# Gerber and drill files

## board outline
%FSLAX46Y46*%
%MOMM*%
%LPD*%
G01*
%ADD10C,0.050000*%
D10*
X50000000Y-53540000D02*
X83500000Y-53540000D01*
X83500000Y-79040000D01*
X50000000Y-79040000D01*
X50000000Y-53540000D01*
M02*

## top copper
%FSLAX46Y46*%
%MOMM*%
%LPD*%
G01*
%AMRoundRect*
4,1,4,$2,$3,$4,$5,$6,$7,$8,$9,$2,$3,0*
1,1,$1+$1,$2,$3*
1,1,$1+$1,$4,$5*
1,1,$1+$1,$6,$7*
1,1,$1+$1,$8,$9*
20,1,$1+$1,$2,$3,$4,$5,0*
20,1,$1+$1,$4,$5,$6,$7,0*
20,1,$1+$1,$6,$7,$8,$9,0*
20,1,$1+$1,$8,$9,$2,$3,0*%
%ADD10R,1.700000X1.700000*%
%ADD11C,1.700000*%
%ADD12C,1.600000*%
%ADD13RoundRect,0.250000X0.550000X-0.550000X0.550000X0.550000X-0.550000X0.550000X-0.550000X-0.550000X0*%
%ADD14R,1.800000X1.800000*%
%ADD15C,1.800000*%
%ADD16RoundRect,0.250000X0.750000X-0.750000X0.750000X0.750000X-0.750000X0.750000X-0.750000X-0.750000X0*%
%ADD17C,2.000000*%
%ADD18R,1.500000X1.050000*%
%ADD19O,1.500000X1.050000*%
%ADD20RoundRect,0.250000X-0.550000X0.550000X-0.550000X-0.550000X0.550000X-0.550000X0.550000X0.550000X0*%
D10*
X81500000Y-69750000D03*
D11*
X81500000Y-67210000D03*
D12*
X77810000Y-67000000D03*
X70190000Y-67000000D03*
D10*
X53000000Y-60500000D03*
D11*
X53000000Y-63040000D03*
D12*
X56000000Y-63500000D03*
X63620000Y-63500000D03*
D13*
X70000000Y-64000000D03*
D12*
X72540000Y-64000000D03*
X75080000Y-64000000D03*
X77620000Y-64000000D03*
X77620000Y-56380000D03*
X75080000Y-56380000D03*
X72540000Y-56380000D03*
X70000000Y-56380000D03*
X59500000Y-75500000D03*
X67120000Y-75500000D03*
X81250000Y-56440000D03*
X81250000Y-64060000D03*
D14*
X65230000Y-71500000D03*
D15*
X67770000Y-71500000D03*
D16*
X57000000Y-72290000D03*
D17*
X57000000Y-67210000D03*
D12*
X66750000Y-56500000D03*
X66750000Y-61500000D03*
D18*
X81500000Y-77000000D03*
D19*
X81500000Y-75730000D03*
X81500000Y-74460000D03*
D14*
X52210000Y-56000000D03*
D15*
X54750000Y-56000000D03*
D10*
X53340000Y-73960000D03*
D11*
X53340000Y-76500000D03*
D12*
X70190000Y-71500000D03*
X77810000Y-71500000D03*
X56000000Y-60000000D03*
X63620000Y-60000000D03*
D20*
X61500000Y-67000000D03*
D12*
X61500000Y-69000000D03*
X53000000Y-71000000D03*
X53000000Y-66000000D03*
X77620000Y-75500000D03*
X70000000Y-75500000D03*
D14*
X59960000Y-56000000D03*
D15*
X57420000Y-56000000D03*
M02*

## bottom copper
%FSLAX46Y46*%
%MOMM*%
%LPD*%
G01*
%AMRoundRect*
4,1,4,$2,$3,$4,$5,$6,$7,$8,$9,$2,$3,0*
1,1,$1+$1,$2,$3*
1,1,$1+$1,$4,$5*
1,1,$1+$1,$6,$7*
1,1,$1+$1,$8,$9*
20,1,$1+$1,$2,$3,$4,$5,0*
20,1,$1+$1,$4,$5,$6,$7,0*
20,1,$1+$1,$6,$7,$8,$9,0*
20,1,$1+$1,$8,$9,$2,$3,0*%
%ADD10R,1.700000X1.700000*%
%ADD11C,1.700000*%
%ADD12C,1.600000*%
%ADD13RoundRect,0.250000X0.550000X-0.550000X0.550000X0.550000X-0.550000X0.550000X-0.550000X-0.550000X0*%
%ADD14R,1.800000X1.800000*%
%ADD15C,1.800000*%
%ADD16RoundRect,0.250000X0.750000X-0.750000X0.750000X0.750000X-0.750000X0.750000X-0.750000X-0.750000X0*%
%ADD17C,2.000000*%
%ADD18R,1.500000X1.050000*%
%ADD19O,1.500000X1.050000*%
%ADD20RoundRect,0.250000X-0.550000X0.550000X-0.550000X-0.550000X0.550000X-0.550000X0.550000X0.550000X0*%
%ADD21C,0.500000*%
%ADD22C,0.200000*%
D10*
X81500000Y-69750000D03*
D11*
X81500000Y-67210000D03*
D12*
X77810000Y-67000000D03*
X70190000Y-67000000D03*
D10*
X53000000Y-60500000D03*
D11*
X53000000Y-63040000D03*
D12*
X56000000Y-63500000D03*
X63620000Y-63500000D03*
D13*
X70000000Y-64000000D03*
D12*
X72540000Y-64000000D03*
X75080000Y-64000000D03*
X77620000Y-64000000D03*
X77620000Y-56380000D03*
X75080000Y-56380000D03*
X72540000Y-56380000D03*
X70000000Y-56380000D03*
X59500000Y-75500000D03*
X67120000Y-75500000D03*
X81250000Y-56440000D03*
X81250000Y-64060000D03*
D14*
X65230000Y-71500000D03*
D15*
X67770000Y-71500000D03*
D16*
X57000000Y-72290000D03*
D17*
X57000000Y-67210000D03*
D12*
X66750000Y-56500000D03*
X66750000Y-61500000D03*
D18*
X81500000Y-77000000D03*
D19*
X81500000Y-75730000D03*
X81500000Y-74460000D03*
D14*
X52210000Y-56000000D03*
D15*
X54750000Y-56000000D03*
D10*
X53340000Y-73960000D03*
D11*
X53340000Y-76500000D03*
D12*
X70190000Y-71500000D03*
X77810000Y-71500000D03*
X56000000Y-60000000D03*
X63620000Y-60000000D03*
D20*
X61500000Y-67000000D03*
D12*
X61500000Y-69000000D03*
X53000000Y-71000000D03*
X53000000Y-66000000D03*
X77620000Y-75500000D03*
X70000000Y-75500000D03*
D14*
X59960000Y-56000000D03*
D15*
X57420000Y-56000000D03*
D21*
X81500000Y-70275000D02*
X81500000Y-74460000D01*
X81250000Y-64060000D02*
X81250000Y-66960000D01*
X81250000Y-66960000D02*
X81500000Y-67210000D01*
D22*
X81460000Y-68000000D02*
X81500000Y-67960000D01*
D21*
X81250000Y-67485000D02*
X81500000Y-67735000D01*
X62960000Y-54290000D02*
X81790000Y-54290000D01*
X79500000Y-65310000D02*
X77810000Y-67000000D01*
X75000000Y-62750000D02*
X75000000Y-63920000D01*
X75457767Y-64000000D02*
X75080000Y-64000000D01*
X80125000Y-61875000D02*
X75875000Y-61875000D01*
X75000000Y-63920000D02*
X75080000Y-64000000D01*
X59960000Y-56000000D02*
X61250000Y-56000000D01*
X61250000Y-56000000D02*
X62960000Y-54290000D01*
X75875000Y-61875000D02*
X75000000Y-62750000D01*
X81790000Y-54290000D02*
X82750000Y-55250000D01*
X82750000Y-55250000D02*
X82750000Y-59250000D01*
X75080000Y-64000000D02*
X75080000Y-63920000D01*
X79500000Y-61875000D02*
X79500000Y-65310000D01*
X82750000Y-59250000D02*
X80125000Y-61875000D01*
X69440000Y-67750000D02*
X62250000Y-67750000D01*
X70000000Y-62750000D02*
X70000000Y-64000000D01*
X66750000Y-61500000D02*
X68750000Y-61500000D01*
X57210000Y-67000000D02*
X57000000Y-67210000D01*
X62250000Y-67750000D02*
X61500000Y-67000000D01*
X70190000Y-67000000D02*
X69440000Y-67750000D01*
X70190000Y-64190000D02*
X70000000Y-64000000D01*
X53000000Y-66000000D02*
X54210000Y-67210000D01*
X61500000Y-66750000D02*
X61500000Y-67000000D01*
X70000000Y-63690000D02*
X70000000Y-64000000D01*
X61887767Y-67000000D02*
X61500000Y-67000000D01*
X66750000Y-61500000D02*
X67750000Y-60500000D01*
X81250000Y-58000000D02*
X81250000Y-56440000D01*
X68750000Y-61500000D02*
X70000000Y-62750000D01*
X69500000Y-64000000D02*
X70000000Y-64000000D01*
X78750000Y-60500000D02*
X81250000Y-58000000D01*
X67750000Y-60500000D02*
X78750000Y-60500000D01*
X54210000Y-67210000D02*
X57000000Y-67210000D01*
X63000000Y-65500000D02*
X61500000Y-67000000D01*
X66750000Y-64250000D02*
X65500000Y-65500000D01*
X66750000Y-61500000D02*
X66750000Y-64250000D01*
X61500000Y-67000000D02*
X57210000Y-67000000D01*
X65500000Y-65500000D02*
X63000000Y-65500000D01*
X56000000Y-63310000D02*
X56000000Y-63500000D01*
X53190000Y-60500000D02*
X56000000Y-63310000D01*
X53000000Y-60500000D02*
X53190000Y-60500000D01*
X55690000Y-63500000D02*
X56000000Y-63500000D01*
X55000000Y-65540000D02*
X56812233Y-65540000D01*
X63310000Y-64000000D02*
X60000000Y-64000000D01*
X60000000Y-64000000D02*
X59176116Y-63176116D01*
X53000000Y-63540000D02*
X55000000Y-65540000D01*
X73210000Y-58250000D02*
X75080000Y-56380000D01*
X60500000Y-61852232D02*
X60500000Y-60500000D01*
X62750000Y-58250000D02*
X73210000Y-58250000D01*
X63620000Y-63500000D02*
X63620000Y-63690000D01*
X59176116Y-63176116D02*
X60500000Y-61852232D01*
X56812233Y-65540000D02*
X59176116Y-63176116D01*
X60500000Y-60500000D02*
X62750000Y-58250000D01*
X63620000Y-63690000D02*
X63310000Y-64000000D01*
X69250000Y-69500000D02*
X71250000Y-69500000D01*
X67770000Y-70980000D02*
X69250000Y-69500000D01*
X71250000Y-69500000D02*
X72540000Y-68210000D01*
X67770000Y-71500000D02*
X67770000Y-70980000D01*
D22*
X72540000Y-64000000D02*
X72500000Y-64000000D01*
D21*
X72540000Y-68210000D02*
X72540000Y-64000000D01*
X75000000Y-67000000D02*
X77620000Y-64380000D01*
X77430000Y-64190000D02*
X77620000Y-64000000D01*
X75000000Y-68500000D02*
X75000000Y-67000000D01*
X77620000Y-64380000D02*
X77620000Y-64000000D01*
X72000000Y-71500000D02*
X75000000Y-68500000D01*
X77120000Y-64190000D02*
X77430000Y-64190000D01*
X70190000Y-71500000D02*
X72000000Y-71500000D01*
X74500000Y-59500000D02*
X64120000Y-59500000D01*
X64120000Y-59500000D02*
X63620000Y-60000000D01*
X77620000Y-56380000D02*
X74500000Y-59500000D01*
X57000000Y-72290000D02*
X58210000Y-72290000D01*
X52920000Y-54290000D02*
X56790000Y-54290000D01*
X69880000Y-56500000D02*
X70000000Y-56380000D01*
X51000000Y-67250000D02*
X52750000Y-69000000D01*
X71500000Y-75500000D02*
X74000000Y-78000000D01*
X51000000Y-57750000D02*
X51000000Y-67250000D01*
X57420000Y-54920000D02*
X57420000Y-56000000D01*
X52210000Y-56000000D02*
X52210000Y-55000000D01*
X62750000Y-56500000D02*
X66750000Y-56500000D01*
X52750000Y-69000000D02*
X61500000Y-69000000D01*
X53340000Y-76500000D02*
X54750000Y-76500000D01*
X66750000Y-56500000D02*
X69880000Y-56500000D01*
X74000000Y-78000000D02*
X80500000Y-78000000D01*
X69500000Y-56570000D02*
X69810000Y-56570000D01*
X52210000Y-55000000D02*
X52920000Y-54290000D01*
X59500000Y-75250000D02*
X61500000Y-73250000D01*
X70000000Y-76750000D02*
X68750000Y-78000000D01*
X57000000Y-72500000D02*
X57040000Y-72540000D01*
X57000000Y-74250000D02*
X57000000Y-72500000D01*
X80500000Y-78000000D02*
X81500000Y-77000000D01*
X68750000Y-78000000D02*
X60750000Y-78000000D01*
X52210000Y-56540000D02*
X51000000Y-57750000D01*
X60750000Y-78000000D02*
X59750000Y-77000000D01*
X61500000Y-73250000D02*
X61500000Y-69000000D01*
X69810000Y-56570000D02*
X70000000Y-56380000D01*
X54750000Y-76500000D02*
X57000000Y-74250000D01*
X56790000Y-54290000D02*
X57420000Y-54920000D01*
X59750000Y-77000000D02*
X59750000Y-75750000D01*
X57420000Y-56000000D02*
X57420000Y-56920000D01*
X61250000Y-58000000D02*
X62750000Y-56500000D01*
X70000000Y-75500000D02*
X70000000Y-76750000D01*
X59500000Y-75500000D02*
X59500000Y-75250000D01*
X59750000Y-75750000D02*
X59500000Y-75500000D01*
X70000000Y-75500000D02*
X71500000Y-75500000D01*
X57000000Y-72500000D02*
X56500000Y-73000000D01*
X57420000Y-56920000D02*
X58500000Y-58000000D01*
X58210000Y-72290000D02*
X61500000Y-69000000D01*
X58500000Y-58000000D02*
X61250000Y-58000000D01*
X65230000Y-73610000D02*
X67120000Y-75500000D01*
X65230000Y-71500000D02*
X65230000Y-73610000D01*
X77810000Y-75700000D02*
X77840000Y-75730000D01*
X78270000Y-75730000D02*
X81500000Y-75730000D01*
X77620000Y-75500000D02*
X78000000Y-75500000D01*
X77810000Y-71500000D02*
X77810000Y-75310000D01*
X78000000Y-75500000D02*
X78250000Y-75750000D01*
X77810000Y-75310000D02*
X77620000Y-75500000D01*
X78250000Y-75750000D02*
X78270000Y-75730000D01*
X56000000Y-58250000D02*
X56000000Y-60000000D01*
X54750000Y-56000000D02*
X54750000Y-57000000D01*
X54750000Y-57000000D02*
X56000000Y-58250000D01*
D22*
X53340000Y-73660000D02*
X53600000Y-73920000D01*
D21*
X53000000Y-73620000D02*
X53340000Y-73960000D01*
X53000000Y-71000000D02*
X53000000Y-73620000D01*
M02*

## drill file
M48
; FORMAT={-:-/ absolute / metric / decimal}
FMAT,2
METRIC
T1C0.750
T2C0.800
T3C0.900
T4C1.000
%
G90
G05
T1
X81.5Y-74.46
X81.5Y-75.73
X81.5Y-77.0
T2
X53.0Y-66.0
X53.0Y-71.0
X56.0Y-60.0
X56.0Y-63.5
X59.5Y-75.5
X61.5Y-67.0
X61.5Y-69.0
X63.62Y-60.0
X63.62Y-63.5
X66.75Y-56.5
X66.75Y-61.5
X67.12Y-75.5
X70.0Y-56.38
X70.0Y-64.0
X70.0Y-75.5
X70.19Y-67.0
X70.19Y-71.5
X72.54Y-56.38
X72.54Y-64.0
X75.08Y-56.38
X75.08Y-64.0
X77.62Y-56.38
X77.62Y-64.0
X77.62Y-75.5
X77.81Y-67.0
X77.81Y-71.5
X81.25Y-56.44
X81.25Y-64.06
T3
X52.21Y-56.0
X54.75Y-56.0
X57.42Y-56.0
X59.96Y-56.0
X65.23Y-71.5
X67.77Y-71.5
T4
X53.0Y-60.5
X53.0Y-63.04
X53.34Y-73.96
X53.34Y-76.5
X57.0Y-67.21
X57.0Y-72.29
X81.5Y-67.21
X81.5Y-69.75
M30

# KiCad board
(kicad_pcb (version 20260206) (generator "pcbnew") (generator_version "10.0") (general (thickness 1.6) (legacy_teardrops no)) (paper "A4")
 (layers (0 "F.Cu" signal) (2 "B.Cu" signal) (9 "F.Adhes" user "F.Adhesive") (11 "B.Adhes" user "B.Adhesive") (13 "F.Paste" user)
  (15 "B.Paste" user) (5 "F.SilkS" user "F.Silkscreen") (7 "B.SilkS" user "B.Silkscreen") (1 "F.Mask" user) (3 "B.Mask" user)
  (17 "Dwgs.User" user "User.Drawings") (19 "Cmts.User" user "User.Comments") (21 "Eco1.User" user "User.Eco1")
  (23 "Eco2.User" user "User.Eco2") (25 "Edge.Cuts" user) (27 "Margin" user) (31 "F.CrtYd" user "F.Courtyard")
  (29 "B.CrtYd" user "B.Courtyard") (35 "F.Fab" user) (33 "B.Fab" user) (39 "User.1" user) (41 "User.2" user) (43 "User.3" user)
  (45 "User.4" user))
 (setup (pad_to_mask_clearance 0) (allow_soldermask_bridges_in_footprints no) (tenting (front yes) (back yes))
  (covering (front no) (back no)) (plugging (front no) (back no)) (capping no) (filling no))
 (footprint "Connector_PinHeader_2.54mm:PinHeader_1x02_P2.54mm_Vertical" (layer "F.Cu") (at 81.5 69.75 180)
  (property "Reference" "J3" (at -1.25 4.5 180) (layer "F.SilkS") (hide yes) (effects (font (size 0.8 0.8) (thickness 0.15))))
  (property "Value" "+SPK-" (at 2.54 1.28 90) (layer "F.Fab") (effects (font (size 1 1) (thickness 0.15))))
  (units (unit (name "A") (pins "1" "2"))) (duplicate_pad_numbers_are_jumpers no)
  (pad "1" thru_hole rect (at 0 0 180) (size 1.7 1.7) (drill 1) (layers "*.Cu" "*.Mask") (remove_unused_layers no) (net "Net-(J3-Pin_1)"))
  (pad "2" thru_hole circle (at 0 2.54 180) (size 1.7 1.7) (drill 1) (layers "*.Cu" "*.Mask") (remove_unused_layers no)
   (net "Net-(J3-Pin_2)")))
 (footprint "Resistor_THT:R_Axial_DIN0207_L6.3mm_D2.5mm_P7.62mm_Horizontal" (layer "F.Cu") (at 77.81 67 180)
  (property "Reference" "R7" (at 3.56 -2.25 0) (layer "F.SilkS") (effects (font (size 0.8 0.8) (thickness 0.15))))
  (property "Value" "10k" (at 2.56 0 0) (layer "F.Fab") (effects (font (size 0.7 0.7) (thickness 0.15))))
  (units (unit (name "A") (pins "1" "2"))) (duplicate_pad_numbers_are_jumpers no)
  (pad "1" thru_hole circle (at 0 0 180) (size 1.6 1.6) (drill 0.8) (layers "*.Cu" "*.Mask") (remove_unused_layers no) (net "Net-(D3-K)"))
  (pad "2" thru_hole circle (at 7.62 0 180) (size 1.6 1.6) (drill 0.8) (layers "*.Cu" "*.Mask") (remove_unused_layers no)
   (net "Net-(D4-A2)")))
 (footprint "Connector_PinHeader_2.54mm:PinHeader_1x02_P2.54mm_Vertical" (layer "F.Cu") (at 53 60.5)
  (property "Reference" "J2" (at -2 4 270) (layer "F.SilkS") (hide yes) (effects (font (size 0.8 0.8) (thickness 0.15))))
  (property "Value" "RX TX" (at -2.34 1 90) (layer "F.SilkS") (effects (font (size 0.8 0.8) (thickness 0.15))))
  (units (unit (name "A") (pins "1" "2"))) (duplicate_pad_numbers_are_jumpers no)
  (pad "1" thru_hole rect (at 0 0) (size 1.7 1.7) (drill 1) (layers "*.Cu" "*.Mask") (remove_unused_layers no) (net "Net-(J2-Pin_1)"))
  (pad "2" thru_hole circle (at 0 2.54) (size 1.7 1.7) (drill 1) (layers "*.Cu" "*.Mask") (remove_unused_layers no) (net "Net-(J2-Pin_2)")))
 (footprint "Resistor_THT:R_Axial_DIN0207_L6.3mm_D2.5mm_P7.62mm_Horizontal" (layer "F.Cu") (at 56 63.5)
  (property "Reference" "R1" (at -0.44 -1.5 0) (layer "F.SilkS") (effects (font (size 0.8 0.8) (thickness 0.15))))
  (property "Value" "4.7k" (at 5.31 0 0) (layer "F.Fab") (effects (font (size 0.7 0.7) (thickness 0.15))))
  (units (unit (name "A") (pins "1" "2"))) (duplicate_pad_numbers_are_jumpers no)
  (pad "1" thru_hole circle (at 0 0) (size 1.6 1.6) (drill 0.8) (layers "*.Cu" "*.Mask") (remove_unused_layers no) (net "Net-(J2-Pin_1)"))
  (pad "2" thru_hole circle (at 7.62 0) (size 1.6 1.6) (drill 0.8) (layers "*.Cu" "*.Mask") (remove_unused_layers no) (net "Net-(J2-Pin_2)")))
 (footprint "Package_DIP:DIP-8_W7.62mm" (layer "F.Cu") (at 70 64 90)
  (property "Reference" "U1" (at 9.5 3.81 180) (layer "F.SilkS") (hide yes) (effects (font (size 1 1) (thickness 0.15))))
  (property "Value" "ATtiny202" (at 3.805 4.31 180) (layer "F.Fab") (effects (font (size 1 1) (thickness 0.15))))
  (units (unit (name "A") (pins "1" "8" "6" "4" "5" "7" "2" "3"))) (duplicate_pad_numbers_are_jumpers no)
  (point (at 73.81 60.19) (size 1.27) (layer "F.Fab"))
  (pad "1" thru_hole roundrect (at 0 0 90) (size 1.6 1.6) (drill 0.8) (layers "*.Cu" "*.Mask") (remove_unused_layers no)
   (roundrect_rratio 0.15625) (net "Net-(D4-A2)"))
  (pad "2" thru_hole circle (at 0 2.54 90) (size 1.6 1.6) (drill 0.8) (layers "*.Cu" "*.Mask") (remove_unused_layers no) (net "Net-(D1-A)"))
  (pad "3" thru_hole circle (at 0 5.08 90) (size 1.6 1.6) (drill 0.8) (layers "*.Cu" "*.Mask") (remove_unused_layers no) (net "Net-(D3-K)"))
  (pad "4" thru_hole circle (at 0 7.62 90) (size 1.6 1.6) (drill 0.8) (layers "*.Cu" "*.Mask") (remove_unused_layers no)
   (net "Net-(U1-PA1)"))
  (pad "5" thru_hole circle (at 7.62 7.62 90) (size 1.6 1.6) (drill 0.8) (layers "*.Cu" "*.Mask") (remove_unused_layers no)
   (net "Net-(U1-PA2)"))
  (pad "6" thru_hole circle (at 7.62 5.08 90) (size 1.6 1.6) (drill 0.8) (layers "*.Cu" "*.Mask") (remove_unused_layers no)
   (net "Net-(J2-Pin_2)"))
  (pad "7" thru_hole circle (at 7.62 2.54 90) (size 1.6 1.6) (drill 0.8) (layers "*.Cu" "*.Mask") (remove_unused_layers no)
   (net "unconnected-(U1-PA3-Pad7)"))
  (pad "8" thru_hole circle (at 7.62 0 90) (size 1.6 1.6) (drill 0.8) (layers "*.Cu" "*.Mask") (remove_unused_layers no) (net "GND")))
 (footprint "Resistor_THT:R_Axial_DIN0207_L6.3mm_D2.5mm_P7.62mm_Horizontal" (layer "F.Cu") (at 59.5 75.5)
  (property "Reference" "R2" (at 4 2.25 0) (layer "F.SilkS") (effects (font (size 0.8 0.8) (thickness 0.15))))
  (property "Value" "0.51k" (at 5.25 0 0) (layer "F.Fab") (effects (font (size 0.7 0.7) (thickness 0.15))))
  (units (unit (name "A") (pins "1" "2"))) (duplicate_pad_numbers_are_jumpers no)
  (pad "1" thru_hole circle (at 0 0) (size 1.6 1.6) (drill 0.8) (layers "*.Cu" "*.Mask") (remove_unused_layers no) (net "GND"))
  (pad "2" thru_hole circle (at 7.62 0) (size 1.6 1.6) (drill 0.8) (layers "*.Cu" "*.Mask") (remove_unused_layers no) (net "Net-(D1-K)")))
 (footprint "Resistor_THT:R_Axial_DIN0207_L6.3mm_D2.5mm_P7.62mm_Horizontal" (layer "F.Cu") (at 81.25 56.44 -90)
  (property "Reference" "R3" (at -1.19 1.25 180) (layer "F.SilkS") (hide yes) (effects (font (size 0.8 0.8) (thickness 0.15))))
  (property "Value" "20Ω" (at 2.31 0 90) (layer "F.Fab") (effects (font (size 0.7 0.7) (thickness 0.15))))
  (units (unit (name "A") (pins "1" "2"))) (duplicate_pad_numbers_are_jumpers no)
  (pad "1" thru_hole circle (at 0 0 270) (size 1.6 1.6) (drill 0.8) (layers "*.Cu" "*.Mask") (remove_unused_layers no) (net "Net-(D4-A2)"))
  (pad "2" thru_hole circle (at 7.62 0 270) (size 1.6 1.6) (drill 0.8) (layers "*.Cu" "*.Mask") (remove_unused_layers no)
   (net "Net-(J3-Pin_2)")))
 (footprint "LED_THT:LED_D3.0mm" (layer "F.Cu") (at 65.23 71.5)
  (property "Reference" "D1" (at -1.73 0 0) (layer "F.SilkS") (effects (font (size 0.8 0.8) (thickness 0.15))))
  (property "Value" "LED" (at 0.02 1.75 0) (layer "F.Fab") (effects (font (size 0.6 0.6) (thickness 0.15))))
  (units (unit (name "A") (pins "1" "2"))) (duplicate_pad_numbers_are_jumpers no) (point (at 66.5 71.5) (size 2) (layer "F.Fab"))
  (pad "1" thru_hole rect (at 0 0) (size 1.8 1.8) (drill 0.9) (layers "*.Cu" "*.Mask") (remove_unused_layers no) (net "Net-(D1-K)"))
  (pad "2" thru_hole circle (at 2.54 0) (size 1.8 1.8) (drill 0.9) (layers "*.Cu" "*.Mask") (remove_unused_layers no) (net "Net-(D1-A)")))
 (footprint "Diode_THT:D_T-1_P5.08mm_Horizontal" (layer "F.Cu") (at 57 72.29 90)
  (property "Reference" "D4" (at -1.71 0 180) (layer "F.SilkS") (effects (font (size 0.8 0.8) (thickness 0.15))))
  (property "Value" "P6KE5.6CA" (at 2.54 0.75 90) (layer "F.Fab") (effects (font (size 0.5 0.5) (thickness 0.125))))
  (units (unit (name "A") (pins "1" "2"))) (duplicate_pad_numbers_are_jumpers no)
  (pad "1" thru_hole roundrect (at 0 0 90) (size 2 2) (drill 1) (layers "*.Cu" "*.Mask") (remove_unused_layers no) (roundrect_rratio 0.125)
   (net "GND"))
  (pad "2" thru_hole circle (at 5.08 0 90) (size 2 2) (drill 1) (layers "*.Cu" "*.Mask") (remove_unused_layers no) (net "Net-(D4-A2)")))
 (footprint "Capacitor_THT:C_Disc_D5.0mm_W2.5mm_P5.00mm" (layer "F.Cu") (at 66.75 56.5 -90)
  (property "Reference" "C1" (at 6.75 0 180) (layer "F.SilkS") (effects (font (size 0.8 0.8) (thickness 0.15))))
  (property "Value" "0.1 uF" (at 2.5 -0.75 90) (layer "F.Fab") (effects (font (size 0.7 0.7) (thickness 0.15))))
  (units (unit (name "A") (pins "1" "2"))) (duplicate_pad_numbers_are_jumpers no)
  (pad "1" thru_hole circle (at 0 0 270) (size 1.6 1.6) (drill 0.8) (layers "*.Cu" "*.Mask") (remove_unused_layers no) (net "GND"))
  (pad "2" thru_hole circle (at 5 0 270) (size 1.6 1.6) (drill 0.8) (layers "*.Cu" "*.Mask") (remove_unused_layers no) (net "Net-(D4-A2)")))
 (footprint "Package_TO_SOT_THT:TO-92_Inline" (layer "F.Cu") (at 81.5 77 90)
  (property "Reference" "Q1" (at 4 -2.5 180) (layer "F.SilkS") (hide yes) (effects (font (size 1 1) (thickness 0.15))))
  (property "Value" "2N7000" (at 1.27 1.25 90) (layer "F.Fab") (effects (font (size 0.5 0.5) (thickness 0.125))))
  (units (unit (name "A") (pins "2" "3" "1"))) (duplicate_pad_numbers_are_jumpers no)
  (pad "1" thru_hole rect (at 0 0 90) (size 1.05 1.5) (drill 0.75) (layers "*.Cu" "*.Mask") (remove_unused_layers no) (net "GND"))
  (pad "2" thru_hole oval (at 1.27 0 90) (size 1.05 1.5) (drill 0.75) (layers "*.Cu" "*.Mask") (remove_unused_layers no) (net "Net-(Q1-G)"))
  (pad "3" thru_hole oval (at 2.54 0 90) (size 1.05 1.5) (drill 0.75) (layers "*.Cu" "*.Mask") (remove_unused_layers no)
   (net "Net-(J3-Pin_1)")))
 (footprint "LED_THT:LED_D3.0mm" (layer "F.Cu") (at 52.21 56)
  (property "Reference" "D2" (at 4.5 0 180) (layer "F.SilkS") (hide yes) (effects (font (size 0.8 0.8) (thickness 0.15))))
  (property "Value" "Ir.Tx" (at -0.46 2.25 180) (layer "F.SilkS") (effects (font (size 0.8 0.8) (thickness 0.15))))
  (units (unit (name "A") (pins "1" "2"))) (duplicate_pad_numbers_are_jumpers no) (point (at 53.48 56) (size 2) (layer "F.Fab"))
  (pad "1" thru_hole rect (at 0 0) (size 1.8 1.8) (drill 0.9) (layers "*.Cu" "*.Mask") (remove_unused_layers no) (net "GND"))
  (pad "2" thru_hole circle (at 2.54 0) (size 1.8 1.8) (drill 0.9) (layers "*.Cu" "*.Mask") (remove_unused_layers no) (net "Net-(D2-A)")))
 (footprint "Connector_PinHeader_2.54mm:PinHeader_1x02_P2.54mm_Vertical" (layer "F.Cu") (at 53.34 73.96)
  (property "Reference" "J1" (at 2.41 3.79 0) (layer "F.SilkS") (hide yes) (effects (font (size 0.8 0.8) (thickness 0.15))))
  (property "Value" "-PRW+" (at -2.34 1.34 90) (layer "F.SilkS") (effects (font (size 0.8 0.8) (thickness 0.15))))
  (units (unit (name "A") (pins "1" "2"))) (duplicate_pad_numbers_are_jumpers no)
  (pad "1" thru_hole rect (at 0 0) (size 1.7 1.7) (drill 1) (layers "*.Cu" "*.Mask") (remove_unused_layers no) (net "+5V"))
  (pad "2" thru_hole circle (at 0 2.54) (size 1.7 1.7) (drill 1) (layers "*.Cu" "*.Mask") (remove_unused_layers no) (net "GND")))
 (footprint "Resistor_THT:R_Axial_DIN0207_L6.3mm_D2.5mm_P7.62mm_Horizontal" (layer "F.Cu") (at 70.19 71.5)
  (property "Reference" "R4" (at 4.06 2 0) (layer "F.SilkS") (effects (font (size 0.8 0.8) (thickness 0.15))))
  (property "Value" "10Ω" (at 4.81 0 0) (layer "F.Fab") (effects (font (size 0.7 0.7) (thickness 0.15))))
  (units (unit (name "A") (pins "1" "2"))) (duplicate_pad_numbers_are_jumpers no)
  (pad "1" thru_hole circle (at 0 0) (size 1.6 1.6) (drill 0.8) (layers "*.Cu" "*.Mask") (remove_unused_layers no) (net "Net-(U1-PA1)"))
  (pad "2" thru_hole circle (at 7.62 0) (size 1.6 1.6) (drill 0.8) (layers "*.Cu" "*.Mask") (remove_unused_layers no) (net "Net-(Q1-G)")))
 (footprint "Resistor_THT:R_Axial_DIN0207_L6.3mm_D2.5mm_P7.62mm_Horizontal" (layer "F.Cu") (at 56 60)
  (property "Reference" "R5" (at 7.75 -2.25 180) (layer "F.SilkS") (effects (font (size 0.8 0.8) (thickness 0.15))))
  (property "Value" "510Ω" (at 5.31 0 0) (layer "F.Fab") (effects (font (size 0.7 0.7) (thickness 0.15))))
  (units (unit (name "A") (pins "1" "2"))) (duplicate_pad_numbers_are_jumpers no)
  (pad "1" thru_hole circle (at 0 0) (size 1.6 1.6) (drill 0.8) (layers "*.Cu" "*.Mask") (remove_unused_layers no) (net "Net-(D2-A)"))
  (pad "2" thru_hole circle (at 7.62 0) (size 1.6 1.6) (drill 0.8) (layers "*.Cu" "*.Mask") (remove_unused_layers no) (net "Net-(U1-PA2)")))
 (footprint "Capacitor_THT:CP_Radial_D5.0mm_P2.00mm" (layer "F.Cu") (at 61.5 67 -90)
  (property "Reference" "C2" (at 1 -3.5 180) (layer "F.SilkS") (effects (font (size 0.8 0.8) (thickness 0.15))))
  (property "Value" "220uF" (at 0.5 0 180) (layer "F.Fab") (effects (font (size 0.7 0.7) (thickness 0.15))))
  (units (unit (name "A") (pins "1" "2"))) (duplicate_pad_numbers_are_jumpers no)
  (pad "1" thru_hole roundrect (at 0 0 270) (size 1.6 1.6) (drill 0.8) (layers "*.Cu" "*.Mask") (remove_unused_layers no)
   (roundrect_rratio 0.15625) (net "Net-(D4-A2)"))
  (pad "2" thru_hole circle (at 2 0 270) (size 1.6 1.6) (drill 0.8) (layers "*.Cu" "*.Mask") (remove_unused_layers no) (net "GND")))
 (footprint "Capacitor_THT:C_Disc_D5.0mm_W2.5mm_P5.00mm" (layer "F.Cu") (at 53 71 90)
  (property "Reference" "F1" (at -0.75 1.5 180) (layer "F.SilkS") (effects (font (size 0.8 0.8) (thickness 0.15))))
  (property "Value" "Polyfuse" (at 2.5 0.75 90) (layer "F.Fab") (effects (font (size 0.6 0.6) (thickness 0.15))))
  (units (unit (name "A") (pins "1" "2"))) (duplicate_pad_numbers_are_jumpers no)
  (pad "1" thru_hole circle (at 0 0 90) (size 1.6 1.6) (drill 0.8) (layers "*.Cu" "*.Mask") (remove_unused_layers no) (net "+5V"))
  (pad "2" thru_hole circle (at 5 0 90) (size 1.6 1.6) (drill 0.8) (layers "*.Cu" "*.Mask") (remove_unused_layers no) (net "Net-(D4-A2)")))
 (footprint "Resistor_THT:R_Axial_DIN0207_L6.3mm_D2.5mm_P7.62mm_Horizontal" (layer "F.Cu") (at 77.62 75.5 180)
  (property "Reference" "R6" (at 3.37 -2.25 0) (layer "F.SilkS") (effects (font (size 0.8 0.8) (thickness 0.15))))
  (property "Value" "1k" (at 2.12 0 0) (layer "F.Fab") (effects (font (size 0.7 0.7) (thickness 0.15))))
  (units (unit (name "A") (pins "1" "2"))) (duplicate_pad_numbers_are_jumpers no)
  (pad "1" thru_hole circle (at 0 0 180) (size 1.6 1.6) (drill 0.8) (layers "*.Cu" "*.Mask") (remove_unused_layers no) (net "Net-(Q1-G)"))
  (pad "2" thru_hole circle (at 7.62 0 180) (size 1.6 1.6) (drill 0.8) (layers "*.Cu" "*.Mask") (remove_unused_layers no) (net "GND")))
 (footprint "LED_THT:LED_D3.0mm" (layer "F.Cu") (at 59.96 56 180)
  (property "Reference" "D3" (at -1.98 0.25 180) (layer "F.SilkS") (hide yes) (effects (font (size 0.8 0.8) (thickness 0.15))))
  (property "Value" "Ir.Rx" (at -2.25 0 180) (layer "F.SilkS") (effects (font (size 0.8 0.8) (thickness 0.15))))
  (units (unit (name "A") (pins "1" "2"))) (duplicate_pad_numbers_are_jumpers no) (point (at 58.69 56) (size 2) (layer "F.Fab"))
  (pad "1" thru_hole rect (at 0 0 180) (size 1.8 1.8) (drill 0.9) (layers "*.Cu" "*.Mask") (remove_unused_layers no) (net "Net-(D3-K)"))
  (pad "2" thru_hole circle (at 2.54 0 180) (size 1.8 1.8) (drill 0.9) (layers "*.Cu" "*.Mask") (remove_unused_layers no) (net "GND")))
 (gr_rect (start 50 53.54) (end 83.5 79.04) (stroke (width 0.05) (type default)) (fill no) (layer "Edge.Cuts"))
 (segment (start 81.5 70.275) (end 81.5 74.46) (width 0.5) (layer "B.Cu") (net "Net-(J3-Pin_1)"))
 (segment (start 81.25 64.06) (end 81.25 66.96) (width 0.5) (layer "B.Cu") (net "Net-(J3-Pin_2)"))
 (segment (start 81.25 66.96) (end 81.5 67.21) (width 0.5) (layer "B.Cu") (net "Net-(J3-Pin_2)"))
 (segment (start 81.46 68) (end 81.5 67.96) (width 0.2) (layer "B.Cu") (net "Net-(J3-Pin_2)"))
 (segment (start 81.25 67.485) (end 81.5 67.735) (width 0.5) (layer "B.Cu") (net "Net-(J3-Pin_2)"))
 (segment (start 62.96 54.29) (end 81.79 54.29) (width 0.5) (layer "B.Cu") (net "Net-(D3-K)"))
 (segment (start 79.5 65.31) (end 77.81 67) (width 0.5) (layer "B.Cu") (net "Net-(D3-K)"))
 (segment (start 75 62.75) (end 75 63.92) (width 0.5) (layer "B.Cu") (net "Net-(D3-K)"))
 (segment (start 75.457767 64) (end 75.08 64) (width 0.5) (layer "B.Cu") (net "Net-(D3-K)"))
 (segment (start 80.125 61.875) (end 75.875 61.875) (width 0.5) (layer "B.Cu") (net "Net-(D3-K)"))
 (segment (start 75 63.92) (end 75.08 64) (width 0.5) (layer "B.Cu") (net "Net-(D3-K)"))
 (segment (start 59.96 56) (end 61.25 56) (width 0.5) (layer "B.Cu") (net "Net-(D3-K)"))
 (segment (start 61.25 56) (end 62.96 54.29) (width 0.5) (layer "B.Cu") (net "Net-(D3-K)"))
 (segment (start 75.875 61.875) (end 75 62.75) (width 0.5) (layer "B.Cu") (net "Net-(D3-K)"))
 (segment (start 81.79 54.29) (end 82.75 55.25) (width 0.5) (layer "B.Cu") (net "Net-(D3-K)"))
 (segment (start 82.75 55.25) (end 82.75 59.25) (width 0.5) (layer "B.Cu") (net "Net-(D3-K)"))
 (segment (start 75.08 64) (end 75.08 63.92) (width 0.5) (layer "B.Cu") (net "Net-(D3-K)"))
 (segment (start 79.5 61.875) (end 79.5 65.31) (width 0.5) (layer "B.Cu") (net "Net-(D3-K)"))
 (segment (start 82.75 59.25) (end 80.125 61.875) (width 0.5) (layer "B.Cu") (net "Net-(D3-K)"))
 (segment (start 69.44 67.75) (end 62.25 67.75) (width 0.5) (layer "B.Cu") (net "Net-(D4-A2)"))
 (segment (start 70 62.75) (end 70 64) (width 0.5) (layer "B.Cu") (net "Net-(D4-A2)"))
 (segment (start 66.75 61.5) (end 68.75 61.5) (width 0.5) (layer "B.Cu") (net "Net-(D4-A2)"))
 (segment (start 57.21 67) (end 57 67.21) (width 0.5) (layer "B.Cu") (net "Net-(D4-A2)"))
 (segment (start 62.25 67.75) (end 61.5 67) (width 0.5) (layer "B.Cu") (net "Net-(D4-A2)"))
 (segment (start 70.19 67) (end 69.44 67.75) (width 0.5) (layer "B.Cu") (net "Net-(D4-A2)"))
 (segment (start 70.19 64.19) (end 70 64) (width 0.5) (layer "B.Cu") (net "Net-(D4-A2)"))
 (segment (start 53 66) (end 54.21 67.21) (width 0.5) (layer "B.Cu") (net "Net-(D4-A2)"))
 (segment (start 61.5 66.75) (end 61.5 67) (width 0.5) (layer "B.Cu") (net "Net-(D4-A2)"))
 (segment (start 70 63.69) (end 70 64) (width 0.5) (layer "B.Cu") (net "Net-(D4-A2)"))
 (segment (start 61.887767 67) (end 61.5 67) (width 0.5) (layer "B.Cu") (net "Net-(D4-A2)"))
 (segment (start 66.75 61.5) (end 67.75 60.5) (width 0.5) (layer "B.Cu") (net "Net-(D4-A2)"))
 (segment (start 81.25 58) (end 81.25 56.44) (width 0.5) (layer "B.Cu") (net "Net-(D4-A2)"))
 (segment (start 68.75 61.5) (end 70 62.75) (width 0.5) (layer "B.Cu") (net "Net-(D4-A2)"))
 (segment (start 69.5 64) (end 70 64) (width 0.5) (layer "B.Cu") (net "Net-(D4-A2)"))
 (segment (start 78.75 60.5) (end 81.25 58) (width 0.5) (layer "B.Cu") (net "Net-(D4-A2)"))
 (segment (start 67.75 60.5) (end 78.75 60.5) (width 0.5) (layer "B.Cu") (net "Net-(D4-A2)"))
 (segment (start 54.21 67.21) (end 57 67.21) (width 0.5) (layer "B.Cu") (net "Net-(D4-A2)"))
 (segment (start 63 65.5) (end 61.5 67) (width 0.5) (layer "B.Cu") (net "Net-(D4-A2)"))
 (segment (start 66.75 64.25) (end 65.5 65.5) (width 0.5) (layer "B.Cu") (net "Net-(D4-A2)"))
 (segment (start 66.75 61.5) (end 66.75 64.25) (width 0.5) (layer "B.Cu") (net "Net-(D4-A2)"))
 (segment (start 61.5 67) (end 57.21 67) (width 0.5) (layer "B.Cu") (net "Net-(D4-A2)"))
 (segment (start 65.5 65.5) (end 63 65.5) (width 0.5) (layer "B.Cu") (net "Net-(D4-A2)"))
 (segment (start 56 63.31) (end 56 63.5) (width 0.5) (layer "B.Cu") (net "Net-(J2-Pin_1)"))
 (segment (start 53.19 60.5) (end 56 63.31) (width 0.5) (layer "B.Cu") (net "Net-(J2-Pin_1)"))
 (segment (start 53 60.5) (end 53.19 60.5) (width 0.5) (layer "B.Cu") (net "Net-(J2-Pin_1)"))
 (segment (start 55.69 63.5) (end 56 63.5) (width 0.5) (layer "B.Cu") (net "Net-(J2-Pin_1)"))
 (segment (start 55 65.54) (end 56.812233 65.54) (width 0.5) (layer "B.Cu") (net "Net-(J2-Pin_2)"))
 (segment (start 63.31 64) (end 60 64) (width 0.5) (layer "B.Cu") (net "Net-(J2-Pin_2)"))
 (segment (start 60 64) (end 59.176116 63.176116) (width 0.5) (layer "B.Cu") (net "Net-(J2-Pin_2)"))
 (segment (start 53 63.54) (end 55 65.54) (width 0.5) (layer "B.Cu") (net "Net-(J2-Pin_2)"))
 (segment (start 73.21 58.25) (end 75.08 56.38) (width 0.5) (layer "B.Cu") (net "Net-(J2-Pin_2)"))
 (segment (start 60.5 61.852232) (end 60.5 60.5) (width 0.5) (layer "B.Cu") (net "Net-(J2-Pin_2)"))
 (segment (start 62.75 58.25) (end 73.21 58.25) (width 0.5) (layer "B.Cu") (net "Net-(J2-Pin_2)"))
 (segment (start 63.62 63.5) (end 63.62 63.69) (width 0.5) (layer "B.Cu") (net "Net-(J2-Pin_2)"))
 (segment (start 59.176116 63.176116) (end 60.5 61.852232) (width 0.5) (layer "B.Cu") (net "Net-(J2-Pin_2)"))
 (segment (start 56.812233 65.54) (end 59.176116 63.176116) (width 0.5) (layer "B.Cu") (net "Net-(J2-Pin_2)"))
 (segment (start 60.5 60.5) (end 62.75 58.25) (width 0.5) (layer "B.Cu") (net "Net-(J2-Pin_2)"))
 (segment (start 63.62 63.69) (end 63.31 64) (width 0.5) (layer "B.Cu") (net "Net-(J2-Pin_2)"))
 (segment (start 69.25 69.5) (end 71.25 69.5) (width 0.5) (layer "B.Cu") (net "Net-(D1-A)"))
 (segment (start 67.77 70.98) (end 69.25 69.5) (width 0.5) (layer "B.Cu") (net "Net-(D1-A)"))
 (segment (start 71.25 69.5) (end 72.54 68.21) (width 0.5) (layer "B.Cu") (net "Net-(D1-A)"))
 (segment (start 67.77 71.5) (end 67.77 70.98) (width 0.5) (layer "B.Cu") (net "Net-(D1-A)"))
 (segment (start 72.54 64) (end 72.5 64) (width 0.2) (layer "B.Cu") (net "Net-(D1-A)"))
 (segment (start 72.54 68.21) (end 72.54 64) (width 0.5) (layer "B.Cu") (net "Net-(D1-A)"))
 (segment (start 75 67) (end 77.62 64.38) (width 0.5) (layer "B.Cu") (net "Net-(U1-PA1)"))
 (segment (start 77.43 64.19) (end 77.62 64) (width 0.5) (layer "B.Cu") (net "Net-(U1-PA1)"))
 (segment (start 75 68.5) (end 75 67) (width 0.5) (layer "B.Cu") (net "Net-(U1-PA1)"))
 (segment (start 77.62 64.38) (end 77.62 64) (width 0.5) (layer "B.Cu") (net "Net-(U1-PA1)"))
 (segment (start 72 71.5) (end 75 68.5) (width 0.5) (layer "B.Cu") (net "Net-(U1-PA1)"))
 (segment (start 77.12 64.19) (end 77.43 64.19) (width 0.5) (layer "B.Cu") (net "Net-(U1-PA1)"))
 (segment (start 70.19 71.5) (end 72 71.5) (width 0.5) (layer "B.Cu") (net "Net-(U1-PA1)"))
 (segment (start 74.5 59.5) (end 64.12 59.5) (width 0.5) (layer "B.Cu") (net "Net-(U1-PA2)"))
 (segment (start 64.12 59.5) (end 63.62 60) (width 0.5) (layer "B.Cu") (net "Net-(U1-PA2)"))
 (segment (start 77.62 56.38) (end 74.5 59.5) (width 0.5) (layer "B.Cu") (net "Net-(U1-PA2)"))
 (segment (start 57 72.29) (end 58.21 72.29) (width 0.5) (layer "B.Cu") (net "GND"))
 (segment (start 52.92 54.29) (end 56.79 54.29) (width 0.5) (layer "B.Cu") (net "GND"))
 (segment (start 69.88 56.5) (end 70 56.38) (width 0.5) (layer "B.Cu") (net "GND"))
 (segment (start 51 67.25) (end 52.75 69) (width 0.5) (layer "B.Cu") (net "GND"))
 (segment (start 71.5 75.5) (end 74 78) (width 0.5) (layer "B.Cu") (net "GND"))
 (segment (start 51 57.75) (end 51 67.25) (width 0.5) (layer "B.Cu") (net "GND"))
 (segment (start 57.42 54.92) (end 57.42 56) (width 0.5) (layer "B.Cu") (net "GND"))
 (segment (start 52.21 56) (end 52.21 55) (width 0.5) (layer "B.Cu") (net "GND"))
 (segment (start 62.75 56.5) (end 66.75 56.5) (width 0.5) (layer "B.Cu") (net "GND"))
 (segment (start 52.75 69) (end 61.5 69) (width 0.5) (layer "B.Cu") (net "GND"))
 (segment (start 53.34 76.5) (end 54.75 76.5) (width 0.5) (layer "B.Cu") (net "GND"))
 (segment (start 66.75 56.5) (end 69.88 56.5) (width 0.5) (layer "B.Cu") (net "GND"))
 (segment (start 74 78) (end 80.5 78) (width 0.5) (layer "B.Cu") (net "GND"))
 (segment (start 69.5 56.57) (end 69.81 56.57) (width 0.5) (layer "B.Cu") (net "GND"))
 (segment (start 52.21 55) (end 52.92 54.29) (width 0.5) (layer "B.Cu") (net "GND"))
 (segment (start 59.5 75.25) (end 61.5 73.25) (width 0.5) (layer "B.Cu") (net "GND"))
 (segment (start 70 76.75) (end 68.75 78) (width 0.5) (layer "B.Cu") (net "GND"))
 (segment (start 57 72.5) (end 57.04 72.54) (width 0.5) (layer "B.Cu") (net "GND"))
 (segment (start 57 74.25) (end 57 72.5) (width 0.5) (layer "B.Cu") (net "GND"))
 (segment (start 80.5 78) (end 81.5 77) (width 0.5) (layer "B.Cu") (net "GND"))
 (segment (start 68.75 78) (end 60.75 78) (width 0.5) (layer "B.Cu") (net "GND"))
 (segment (start 52.21 56.54) (end 51 57.75) (width 0.5) (layer "B.Cu") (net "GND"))
 (segment (start 60.75 78) (end 59.75 77) (width 0.5) (layer "B.Cu") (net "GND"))
 (segment (start 61.5 73.25) (end 61.5 69) (width 0.5) (layer "B.Cu") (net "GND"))
 (segment (start 69.81 56.57) (end 70 56.38) (width 0.5) (layer "B.Cu") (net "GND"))
 (segment (start 54.75 76.5) (end 57 74.25) (width 0.5) (layer "B.Cu") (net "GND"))
 (segment (start 56.79 54.29) (end 57.42 54.92) (width 0.5) (layer "B.Cu") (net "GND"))
 (segment (start 59.75 77) (end 59.75 75.75) (width 0.5) (layer "B.Cu") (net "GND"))
 (segment (start 57.42 56) (end 57.42 56.92) (width 0.5) (layer "B.Cu") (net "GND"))
 (segment (start 61.25 58) (end 62.75 56.5) (width 0.5) (layer "B.Cu") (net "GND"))
 (segment (start 70 75.5) (end 70 76.75) (width 0.5) (layer "B.Cu") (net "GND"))
 (segment (start 59.5 75.5) (end 59.5 75.25) (width 0.5) (layer "B.Cu") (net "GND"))
 (segment (start 59.75 75.75) (end 59.5 75.5) (width 0.5) (layer "B.Cu") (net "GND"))
 (segment (start 70 75.5) (end 71.5 75.5) (width 0.5) (layer "B.Cu") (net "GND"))
 (segment (start 57 72.5) (end 56.5 73) (width 0.5) (layer "B.Cu") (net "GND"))
 (segment (start 57.42 56.92) (end 58.5 58) (width 0.5) (layer "B.Cu") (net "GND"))
 (segment (start 58.21 72.29) (end 61.5 69) (width 0.5) (layer "B.Cu") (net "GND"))
 (segment (start 58.5 58) (end 61.25 58) (width 0.5) (layer "B.Cu") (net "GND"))
 (segment (start 65.23 73.61) (end 67.12 75.5) (width 0.5) (layer "B.Cu") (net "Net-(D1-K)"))
 (segment (start 65.23 71.5) (end 65.23 73.61) (width 0.5) (layer "B.Cu") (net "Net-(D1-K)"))
 (segment (start 77.81 75.7) (end 77.84 75.73) (width 0.5) (layer "B.Cu") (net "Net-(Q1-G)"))
 (segment (start 78.27 75.73) (end 81.5 75.73) (width 0.5) (layer "B.Cu") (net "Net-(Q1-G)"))
 (segment (start 77.62 75.5) (end 78 75.5) (width 0.5) (layer "B.Cu") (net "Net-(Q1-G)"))
 (segment (start 77.81 71.5) (end 77.81 75.31) (width 0.5) (layer "B.Cu") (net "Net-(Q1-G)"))
 (segment (start 78 75.5) (end 78.25 75.75) (width 0.5) (layer "B.Cu") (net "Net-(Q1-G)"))
 (segment (start 77.81 75.31) (end 77.62 75.5) (width 0.5) (layer "B.Cu") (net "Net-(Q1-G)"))
 (segment (start 78.25 75.75) (end 78.27 75.73) (width 0.5) (layer "B.Cu") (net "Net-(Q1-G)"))
 (segment (start 56 58.25) (end 56 60) (width 0.5) (layer "B.Cu") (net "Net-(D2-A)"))
 (segment (start 54.75 56) (end 54.75 57) (width 0.5) (layer "B.Cu") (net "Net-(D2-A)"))
 (segment (start 54.75 57) (end 56 58.25) (width 0.5) (layer "B.Cu") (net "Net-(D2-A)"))
 (segment (start 53.34 73.66) (end 53.6 73.92) (width 0.2) (layer "B.Cu") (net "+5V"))
 (segment (start 53 73.62) (end 53.34 73.96) (width 0.5) (layer "B.Cu") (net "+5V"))
 (segment (start 53 71) (end 53 73.62) (width 0.5) (layer "B.Cu") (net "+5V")))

